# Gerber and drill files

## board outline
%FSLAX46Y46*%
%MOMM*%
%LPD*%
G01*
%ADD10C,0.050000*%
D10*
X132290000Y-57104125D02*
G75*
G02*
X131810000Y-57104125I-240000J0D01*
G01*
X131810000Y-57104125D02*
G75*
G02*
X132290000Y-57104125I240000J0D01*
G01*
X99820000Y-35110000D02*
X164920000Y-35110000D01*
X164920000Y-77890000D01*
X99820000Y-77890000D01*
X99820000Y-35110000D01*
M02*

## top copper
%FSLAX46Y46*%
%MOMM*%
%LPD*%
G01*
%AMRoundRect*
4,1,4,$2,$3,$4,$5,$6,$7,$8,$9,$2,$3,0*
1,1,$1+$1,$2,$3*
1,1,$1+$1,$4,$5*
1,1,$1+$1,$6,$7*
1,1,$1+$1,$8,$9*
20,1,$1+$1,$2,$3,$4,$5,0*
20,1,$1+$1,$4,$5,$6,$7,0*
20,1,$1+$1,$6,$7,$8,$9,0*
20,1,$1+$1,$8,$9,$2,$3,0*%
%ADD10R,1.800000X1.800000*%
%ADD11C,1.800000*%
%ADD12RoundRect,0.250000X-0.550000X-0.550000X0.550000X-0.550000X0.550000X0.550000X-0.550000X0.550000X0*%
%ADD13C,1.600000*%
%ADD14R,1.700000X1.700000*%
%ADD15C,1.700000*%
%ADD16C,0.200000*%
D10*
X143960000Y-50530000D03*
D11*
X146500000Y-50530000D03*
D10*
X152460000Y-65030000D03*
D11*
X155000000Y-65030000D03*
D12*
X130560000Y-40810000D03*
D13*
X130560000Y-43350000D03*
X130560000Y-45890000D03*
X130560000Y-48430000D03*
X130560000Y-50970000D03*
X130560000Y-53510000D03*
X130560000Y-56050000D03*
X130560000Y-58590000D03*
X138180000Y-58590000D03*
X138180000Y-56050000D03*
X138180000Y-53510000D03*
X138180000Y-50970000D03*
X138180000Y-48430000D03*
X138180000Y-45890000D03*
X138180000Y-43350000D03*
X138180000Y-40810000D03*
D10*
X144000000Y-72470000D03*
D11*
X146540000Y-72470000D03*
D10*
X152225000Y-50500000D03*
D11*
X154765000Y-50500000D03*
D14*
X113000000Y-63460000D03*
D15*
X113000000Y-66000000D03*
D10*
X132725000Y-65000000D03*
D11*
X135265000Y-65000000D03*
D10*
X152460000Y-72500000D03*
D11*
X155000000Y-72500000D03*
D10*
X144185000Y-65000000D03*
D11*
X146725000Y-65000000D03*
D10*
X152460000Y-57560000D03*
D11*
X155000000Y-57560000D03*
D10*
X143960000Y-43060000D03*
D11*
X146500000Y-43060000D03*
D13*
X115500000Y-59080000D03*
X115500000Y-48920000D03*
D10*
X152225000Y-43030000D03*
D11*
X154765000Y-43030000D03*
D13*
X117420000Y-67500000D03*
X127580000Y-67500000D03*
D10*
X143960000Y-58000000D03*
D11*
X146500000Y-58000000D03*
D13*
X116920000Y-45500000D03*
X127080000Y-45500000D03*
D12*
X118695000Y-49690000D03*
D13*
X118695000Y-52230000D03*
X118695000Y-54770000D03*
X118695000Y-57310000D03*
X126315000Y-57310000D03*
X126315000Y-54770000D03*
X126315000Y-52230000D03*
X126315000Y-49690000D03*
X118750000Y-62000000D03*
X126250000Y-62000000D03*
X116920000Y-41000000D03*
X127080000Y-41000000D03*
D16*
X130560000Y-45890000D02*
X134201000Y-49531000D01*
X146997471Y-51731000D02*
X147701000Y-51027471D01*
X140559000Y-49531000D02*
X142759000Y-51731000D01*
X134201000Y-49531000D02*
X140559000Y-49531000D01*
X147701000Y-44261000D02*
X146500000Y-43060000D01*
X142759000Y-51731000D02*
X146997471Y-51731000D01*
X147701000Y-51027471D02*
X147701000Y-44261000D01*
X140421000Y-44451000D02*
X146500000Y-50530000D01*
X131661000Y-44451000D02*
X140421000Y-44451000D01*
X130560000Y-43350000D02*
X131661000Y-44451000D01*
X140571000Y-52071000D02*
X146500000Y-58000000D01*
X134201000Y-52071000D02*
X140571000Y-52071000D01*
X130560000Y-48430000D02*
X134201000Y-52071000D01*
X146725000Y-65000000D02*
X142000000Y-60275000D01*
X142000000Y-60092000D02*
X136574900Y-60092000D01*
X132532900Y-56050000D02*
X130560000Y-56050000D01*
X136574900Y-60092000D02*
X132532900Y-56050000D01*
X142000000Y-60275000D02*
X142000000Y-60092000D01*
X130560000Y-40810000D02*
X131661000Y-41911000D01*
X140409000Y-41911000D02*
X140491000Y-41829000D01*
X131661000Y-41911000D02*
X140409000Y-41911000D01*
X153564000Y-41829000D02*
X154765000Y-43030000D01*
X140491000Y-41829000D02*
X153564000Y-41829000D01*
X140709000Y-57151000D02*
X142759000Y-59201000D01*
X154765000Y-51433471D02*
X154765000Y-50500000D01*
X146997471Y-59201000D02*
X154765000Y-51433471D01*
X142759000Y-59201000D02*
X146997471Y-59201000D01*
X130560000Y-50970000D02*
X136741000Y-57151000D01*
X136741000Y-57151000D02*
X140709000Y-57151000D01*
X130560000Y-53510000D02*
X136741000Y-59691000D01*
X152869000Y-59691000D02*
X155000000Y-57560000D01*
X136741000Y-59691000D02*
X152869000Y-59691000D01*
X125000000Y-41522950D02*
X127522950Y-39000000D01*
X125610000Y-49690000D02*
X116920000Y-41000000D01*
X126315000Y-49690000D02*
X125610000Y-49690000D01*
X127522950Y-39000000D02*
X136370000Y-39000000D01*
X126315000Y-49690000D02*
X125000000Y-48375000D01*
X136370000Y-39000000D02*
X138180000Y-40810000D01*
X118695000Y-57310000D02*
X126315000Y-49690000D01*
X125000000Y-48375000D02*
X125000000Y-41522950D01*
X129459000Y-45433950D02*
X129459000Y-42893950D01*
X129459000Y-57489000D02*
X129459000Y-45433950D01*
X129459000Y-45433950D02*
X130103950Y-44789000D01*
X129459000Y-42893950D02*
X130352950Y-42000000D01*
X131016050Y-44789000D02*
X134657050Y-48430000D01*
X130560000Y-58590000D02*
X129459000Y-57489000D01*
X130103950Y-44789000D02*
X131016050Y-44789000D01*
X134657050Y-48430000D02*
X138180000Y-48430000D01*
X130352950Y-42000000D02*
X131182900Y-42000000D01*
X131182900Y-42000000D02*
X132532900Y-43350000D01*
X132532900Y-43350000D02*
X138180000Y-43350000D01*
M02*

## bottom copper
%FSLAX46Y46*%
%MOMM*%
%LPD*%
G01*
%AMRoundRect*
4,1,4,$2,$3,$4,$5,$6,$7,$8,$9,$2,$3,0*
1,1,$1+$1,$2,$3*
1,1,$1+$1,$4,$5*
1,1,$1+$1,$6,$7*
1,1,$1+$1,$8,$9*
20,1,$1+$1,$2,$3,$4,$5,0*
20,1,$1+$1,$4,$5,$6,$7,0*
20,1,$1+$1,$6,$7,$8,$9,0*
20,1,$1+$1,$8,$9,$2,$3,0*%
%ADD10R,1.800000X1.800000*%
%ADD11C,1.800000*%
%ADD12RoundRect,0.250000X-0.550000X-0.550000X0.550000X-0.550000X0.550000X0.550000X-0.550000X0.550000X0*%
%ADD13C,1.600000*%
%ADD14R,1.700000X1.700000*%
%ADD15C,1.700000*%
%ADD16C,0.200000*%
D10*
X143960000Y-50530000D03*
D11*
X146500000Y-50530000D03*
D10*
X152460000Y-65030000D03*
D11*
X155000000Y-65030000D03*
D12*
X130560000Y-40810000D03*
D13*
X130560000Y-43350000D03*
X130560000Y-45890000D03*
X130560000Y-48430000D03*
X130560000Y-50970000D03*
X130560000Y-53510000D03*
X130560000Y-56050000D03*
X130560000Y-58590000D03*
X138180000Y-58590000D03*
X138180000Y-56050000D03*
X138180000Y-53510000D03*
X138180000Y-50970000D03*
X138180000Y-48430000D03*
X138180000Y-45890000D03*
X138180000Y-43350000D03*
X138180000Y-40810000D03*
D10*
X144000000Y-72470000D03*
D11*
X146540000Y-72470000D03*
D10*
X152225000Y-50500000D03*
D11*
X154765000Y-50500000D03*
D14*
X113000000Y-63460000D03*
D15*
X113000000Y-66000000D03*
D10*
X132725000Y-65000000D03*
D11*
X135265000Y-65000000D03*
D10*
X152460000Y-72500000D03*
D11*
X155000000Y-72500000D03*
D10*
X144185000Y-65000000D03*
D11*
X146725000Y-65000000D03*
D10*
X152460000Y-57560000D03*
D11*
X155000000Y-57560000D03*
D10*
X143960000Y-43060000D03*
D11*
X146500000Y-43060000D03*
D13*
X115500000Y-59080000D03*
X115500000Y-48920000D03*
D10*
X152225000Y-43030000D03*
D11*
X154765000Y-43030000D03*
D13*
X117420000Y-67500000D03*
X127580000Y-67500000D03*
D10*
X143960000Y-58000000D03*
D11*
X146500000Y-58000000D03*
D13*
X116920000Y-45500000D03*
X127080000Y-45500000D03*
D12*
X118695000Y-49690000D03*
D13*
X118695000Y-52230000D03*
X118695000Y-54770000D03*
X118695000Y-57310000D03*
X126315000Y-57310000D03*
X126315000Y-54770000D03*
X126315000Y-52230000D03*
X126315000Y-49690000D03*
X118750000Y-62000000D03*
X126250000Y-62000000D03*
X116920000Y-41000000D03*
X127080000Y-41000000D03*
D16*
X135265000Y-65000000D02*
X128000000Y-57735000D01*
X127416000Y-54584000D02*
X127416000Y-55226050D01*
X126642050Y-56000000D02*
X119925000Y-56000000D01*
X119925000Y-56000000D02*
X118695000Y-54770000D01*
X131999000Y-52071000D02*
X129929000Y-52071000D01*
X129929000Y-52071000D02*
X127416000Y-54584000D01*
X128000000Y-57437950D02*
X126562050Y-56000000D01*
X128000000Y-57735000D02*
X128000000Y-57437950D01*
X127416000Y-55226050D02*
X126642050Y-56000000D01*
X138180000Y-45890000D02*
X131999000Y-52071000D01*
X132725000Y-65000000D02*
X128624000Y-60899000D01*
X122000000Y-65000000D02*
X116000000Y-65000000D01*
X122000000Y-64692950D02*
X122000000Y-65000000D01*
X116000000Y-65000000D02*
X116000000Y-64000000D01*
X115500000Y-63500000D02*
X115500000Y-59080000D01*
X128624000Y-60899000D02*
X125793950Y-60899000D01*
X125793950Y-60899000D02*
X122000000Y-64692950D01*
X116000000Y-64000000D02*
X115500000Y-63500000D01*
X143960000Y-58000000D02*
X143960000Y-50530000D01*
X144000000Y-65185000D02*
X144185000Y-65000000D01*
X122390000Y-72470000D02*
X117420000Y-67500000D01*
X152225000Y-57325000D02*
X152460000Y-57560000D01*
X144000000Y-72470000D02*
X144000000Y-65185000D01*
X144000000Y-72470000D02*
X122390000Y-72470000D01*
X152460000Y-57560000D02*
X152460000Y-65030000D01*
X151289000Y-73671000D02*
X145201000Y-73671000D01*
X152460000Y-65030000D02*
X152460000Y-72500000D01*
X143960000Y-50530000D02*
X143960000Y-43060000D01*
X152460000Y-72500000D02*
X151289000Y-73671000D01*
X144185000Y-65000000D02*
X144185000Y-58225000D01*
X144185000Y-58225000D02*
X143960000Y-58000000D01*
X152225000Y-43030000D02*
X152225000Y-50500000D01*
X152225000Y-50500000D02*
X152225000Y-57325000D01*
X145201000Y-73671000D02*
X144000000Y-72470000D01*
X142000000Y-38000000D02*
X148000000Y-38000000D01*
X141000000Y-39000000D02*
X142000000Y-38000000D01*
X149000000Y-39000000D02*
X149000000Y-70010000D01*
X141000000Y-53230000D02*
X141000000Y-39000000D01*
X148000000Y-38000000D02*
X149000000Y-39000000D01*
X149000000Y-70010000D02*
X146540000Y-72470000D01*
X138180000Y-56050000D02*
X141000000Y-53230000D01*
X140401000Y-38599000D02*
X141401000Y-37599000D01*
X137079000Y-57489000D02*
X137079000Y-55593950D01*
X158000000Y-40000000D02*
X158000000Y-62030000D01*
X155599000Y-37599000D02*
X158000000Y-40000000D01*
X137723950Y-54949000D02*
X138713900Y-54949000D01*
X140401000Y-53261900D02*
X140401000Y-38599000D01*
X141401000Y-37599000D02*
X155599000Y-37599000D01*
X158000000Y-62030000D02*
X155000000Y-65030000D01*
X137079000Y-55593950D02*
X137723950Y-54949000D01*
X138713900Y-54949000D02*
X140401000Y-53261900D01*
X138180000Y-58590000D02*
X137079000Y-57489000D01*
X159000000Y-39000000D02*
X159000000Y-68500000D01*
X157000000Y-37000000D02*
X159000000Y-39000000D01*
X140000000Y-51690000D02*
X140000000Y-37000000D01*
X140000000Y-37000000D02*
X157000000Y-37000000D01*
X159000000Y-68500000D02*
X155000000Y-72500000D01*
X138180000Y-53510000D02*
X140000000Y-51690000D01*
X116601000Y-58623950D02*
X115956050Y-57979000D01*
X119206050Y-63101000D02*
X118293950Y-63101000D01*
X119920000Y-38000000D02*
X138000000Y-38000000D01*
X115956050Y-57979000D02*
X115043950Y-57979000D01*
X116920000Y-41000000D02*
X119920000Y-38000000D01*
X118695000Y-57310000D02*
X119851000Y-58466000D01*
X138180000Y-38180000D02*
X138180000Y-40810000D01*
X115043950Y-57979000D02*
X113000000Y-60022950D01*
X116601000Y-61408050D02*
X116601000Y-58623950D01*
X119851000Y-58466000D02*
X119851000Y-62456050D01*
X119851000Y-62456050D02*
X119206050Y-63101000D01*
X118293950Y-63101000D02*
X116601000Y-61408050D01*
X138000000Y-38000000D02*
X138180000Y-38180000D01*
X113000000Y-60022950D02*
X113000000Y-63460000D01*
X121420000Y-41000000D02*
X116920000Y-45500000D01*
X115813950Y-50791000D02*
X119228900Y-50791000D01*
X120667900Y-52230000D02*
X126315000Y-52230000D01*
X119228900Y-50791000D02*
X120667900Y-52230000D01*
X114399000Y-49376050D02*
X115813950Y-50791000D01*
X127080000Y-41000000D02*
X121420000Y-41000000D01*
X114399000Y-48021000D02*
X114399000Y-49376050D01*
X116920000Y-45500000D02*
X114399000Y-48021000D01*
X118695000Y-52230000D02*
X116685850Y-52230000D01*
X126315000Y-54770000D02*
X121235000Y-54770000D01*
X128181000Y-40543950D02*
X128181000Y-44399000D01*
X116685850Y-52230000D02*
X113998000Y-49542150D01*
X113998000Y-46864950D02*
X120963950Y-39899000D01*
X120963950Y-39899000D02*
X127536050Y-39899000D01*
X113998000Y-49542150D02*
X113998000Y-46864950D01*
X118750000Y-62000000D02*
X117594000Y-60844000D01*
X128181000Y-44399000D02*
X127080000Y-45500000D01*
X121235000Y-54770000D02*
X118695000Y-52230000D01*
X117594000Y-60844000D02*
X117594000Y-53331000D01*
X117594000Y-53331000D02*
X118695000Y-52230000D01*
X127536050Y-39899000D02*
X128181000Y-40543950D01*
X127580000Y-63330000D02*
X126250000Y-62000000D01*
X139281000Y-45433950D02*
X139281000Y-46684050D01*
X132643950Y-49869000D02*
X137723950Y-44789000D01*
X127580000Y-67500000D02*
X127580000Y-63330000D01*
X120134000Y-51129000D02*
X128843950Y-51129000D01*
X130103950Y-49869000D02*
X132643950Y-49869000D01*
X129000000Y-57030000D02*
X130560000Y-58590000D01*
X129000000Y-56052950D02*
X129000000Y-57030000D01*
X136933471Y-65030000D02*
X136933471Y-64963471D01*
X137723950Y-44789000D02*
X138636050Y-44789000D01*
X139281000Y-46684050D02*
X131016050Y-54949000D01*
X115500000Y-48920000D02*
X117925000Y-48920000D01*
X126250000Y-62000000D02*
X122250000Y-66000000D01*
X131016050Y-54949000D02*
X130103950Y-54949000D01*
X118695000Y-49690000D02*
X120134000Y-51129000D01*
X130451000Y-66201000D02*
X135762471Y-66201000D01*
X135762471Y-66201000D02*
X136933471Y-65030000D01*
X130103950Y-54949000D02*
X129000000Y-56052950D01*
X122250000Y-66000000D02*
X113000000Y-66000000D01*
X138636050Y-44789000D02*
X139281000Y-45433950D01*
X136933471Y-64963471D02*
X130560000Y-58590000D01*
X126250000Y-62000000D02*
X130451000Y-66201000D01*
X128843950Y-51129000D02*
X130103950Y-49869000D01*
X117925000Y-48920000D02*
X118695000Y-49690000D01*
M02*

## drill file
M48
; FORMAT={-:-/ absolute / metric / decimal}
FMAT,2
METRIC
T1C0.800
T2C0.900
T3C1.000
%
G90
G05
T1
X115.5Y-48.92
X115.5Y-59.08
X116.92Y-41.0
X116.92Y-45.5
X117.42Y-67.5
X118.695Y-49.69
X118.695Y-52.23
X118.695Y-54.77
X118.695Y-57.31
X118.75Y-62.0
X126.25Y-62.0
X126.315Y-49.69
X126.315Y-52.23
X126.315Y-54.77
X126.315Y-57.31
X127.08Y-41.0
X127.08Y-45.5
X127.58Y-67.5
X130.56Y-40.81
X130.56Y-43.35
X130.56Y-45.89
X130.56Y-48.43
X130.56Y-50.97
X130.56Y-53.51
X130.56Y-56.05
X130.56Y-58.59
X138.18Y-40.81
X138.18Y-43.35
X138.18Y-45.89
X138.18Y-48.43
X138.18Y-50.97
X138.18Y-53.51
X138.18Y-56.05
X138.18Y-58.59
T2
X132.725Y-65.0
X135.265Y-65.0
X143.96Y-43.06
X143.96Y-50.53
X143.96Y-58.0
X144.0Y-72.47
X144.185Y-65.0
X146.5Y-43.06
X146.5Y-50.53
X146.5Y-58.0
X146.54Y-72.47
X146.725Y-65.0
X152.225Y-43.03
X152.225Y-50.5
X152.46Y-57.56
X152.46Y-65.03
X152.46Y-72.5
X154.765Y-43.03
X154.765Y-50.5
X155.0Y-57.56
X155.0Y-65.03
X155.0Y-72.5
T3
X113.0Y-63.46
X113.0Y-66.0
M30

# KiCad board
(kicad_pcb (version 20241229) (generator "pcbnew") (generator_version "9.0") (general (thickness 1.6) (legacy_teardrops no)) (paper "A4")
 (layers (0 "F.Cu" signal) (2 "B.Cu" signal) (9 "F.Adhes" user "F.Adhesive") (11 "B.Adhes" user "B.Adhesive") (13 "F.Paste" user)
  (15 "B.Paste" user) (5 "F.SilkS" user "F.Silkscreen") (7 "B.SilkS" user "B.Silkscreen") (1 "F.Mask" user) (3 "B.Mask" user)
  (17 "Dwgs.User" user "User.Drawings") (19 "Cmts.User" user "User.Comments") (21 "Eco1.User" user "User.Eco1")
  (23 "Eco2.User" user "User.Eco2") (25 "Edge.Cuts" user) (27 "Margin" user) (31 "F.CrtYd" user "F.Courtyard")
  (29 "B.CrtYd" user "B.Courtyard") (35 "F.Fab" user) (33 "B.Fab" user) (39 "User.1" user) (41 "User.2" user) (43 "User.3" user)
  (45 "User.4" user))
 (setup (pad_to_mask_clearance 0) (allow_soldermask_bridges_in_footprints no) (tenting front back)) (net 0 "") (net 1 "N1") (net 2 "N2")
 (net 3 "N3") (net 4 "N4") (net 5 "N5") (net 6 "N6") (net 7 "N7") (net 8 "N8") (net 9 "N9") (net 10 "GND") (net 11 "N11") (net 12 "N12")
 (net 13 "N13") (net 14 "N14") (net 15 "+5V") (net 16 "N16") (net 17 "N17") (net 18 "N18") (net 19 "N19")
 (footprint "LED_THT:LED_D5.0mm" (layer "F.Cu") (at 143.96 50.53)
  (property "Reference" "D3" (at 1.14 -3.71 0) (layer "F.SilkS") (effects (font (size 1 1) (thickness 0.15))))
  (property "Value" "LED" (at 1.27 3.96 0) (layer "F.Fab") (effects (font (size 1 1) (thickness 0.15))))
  (pad "1" thru_hole rect (at 0 0) (size 1.8 1.8) (drill 0.9) (layers "*.Cu" "*.Mask") (remove_unused_layers no) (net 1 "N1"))
  (pad "2" thru_hole circle (at 2.54 0) (size 1.8 1.8) (drill 0.9) (layers "*.Cu" "*.Mask") (remove_unused_layers no) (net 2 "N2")))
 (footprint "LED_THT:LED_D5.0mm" (layer "F.Cu") (at 152.46 65.03)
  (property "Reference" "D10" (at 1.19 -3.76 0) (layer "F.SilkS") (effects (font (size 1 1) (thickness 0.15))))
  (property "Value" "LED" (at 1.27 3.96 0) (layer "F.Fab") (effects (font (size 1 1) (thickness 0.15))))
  (pad "1" thru_hole rect (at 0 0) (size 1.8 1.8) (drill 0.9) (layers "*.Cu" "*.Mask") (remove_unused_layers no) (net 1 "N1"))
  (pad "2" thru_hole circle (at 2.54 0) (size 1.8 1.8) (drill 0.9) (layers "*.Cu" "*.Mask") (remove_unused_layers no) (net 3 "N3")))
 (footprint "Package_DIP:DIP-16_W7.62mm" (layer "F.Cu") (at 130.56 40.81)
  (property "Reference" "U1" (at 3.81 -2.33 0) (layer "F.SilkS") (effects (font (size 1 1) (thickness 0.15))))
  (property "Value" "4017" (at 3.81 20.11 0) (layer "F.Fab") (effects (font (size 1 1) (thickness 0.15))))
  (pad "1" thru_hole roundrect (at 0 0) (size 1.6 1.6) (drill 0.8) (layers "*.Cu" "*.Mask") (remove_unused_layers no)
   (roundrect_rratio 0.15625) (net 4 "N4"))
  (pad "2" thru_hole circle (at 0 2.54) (size 1.6 1.6) (drill 0.8) (layers "*.Cu" "*.Mask") (remove_unused_layers no) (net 2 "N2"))
  (pad "3" thru_hole circle (at 0 5.08) (size 1.6 1.6) (drill 0.8) (layers "*.Cu" "*.Mask") (remove_unused_layers no) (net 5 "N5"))
  (pad "4" thru_hole circle (at 0 7.62) (size 1.6 1.6) (drill 0.8) (layers "*.Cu" "*.Mask") (remove_unused_layers no) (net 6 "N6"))
  (pad "5" thru_hole circle (at 0 10.16) (size 1.6 1.6) (drill 0.8) (layers "*.Cu" "*.Mask") (remove_unused_layers no) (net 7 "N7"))
  (pad "6" thru_hole circle (at 0 12.7) (size 1.6 1.6) (drill 0.8) (layers "*.Cu" "*.Mask") (remove_unused_layers no) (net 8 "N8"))
  (pad "7" thru_hole circle (at 0 15.24) (size 1.6 1.6) (drill 0.8) (layers "*.Cu" "*.Mask") (remove_unused_layers no) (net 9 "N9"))
  (pad "8" thru_hole circle (at 0 17.78) (size 1.6 1.6) (drill 0.8) (layers "*.Cu" "*.Mask") (remove_unused_layers no) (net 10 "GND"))
  (pad "9" thru_hole circle (at 7.62 17.78) (size 1.6 1.6) (drill 0.8) (layers "*.Cu" "*.Mask") (remove_unused_layers no) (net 3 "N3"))
  (pad "10" thru_hole circle (at 7.62 15.24) (size 1.6 1.6) (drill 0.8) (layers "*.Cu" "*.Mask") (remove_unused_layers no) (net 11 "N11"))
  (pad "11" thru_hole circle (at 7.62 12.7) (size 1.6 1.6) (drill 0.8) (layers "*.Cu" "*.Mask") (remove_unused_layers no) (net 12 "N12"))
  (pad "12" thru_hole circle (at 7.62 10.16) (size 1.6 1.6) (drill 0.8) (layers "*.Cu" "*.Mask") (remove_unused_layers no) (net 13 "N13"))
  (pad "13" thru_hole circle (at 7.62 7.62) (size 1.6 1.6) (drill 0.8) (layers "*.Cu" "*.Mask") (remove_unused_layers no) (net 10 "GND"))
  (pad "14" thru_hole circle (at 7.62 5.08) (size 1.6 1.6) (drill 0.8) (layers "*.Cu" "*.Mask") (remove_unused_layers no) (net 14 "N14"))
  (pad "15" thru_hole circle (at 7.62 2.54) (size 1.6 1.6) (drill 0.8) (layers "*.Cu" "*.Mask") (remove_unused_layers no) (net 10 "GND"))
  (pad "16" thru_hole circle (at 7.62 0) (size 1.6 1.6) (drill 0.8) (layers "*.Cu" "*.Mask") (remove_unused_layers no) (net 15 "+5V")))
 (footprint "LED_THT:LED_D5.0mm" (layer "F.Cu") (at 144 72.47)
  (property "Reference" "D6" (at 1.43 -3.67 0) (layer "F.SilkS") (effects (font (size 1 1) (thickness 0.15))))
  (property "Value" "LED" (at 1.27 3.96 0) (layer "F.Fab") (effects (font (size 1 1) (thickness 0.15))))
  (pad "1" thru_hole rect (at 0 0) (size 1.8 1.8) (drill 0.9) (layers "*.Cu" "*.Mask") (remove_unused_layers no) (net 1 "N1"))
  (pad "2" thru_hole circle (at 2.54 0) (size 1.8 1.8) (drill 0.9) (layers "*.Cu" "*.Mask") (remove_unused_layers no) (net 11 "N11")))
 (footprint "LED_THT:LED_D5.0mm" (layer "F.Cu") (at 152.225 50.5)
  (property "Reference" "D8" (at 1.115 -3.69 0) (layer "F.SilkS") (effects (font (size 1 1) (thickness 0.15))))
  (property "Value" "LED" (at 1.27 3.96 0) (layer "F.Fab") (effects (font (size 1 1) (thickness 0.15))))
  (pad "1" thru_hole rect (at 0 0) (size 1.8 1.8) (drill 0.9) (layers "*.Cu" "*.Mask") (remove_unused_layers no) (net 1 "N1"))
  (pad "2" thru_hole circle (at 2.54 0) (size 1.8 1.8) (drill 0.9) (layers "*.Cu" "*.Mask") (remove_unused_layers no) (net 7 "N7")))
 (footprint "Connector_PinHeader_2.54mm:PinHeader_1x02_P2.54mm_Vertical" (layer "F.Cu") (at 113 63.46)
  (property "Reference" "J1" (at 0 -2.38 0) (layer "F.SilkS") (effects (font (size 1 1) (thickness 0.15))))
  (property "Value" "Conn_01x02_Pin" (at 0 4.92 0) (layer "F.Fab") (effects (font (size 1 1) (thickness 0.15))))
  (pad "1" thru_hole rect (at 0 0) (size 1.7 1.7) (drill 1) (layers "*.Cu" "*.Mask") (remove_unused_layers no) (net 15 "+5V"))
  (pad "2" thru_hole circle (at 0 2.54) (size 1.7 1.7) (drill 1) (layers "*.Cu" "*.Mask") (remove_unused_layers no) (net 10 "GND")))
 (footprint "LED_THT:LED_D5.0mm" (layer "F.Cu") (at 132.725 65)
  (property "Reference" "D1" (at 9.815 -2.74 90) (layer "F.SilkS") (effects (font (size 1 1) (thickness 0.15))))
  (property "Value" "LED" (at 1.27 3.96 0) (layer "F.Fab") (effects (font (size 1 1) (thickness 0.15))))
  (pad "1" thru_hole rect (at 0 0) (size 1.8 1.8) (drill 0.9) (layers "*.Cu" "*.Mask") (remove_unused_layers no) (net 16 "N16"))
  (pad "2" thru_hole circle (at 2.54 0) (size 1.8 1.8) (drill 0.9) (layers "*.Cu" "*.Mask") (remove_unused_layers no) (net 14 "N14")))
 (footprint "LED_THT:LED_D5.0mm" (layer "F.Cu") (at 152.46 72.5)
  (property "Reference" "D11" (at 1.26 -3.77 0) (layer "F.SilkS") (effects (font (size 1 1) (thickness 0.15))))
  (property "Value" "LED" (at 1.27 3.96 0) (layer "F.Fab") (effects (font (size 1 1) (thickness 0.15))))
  (pad "1" thru_hole rect (at 0 0) (size 1.8 1.8) (drill 0.9) (layers "*.Cu" "*.Mask") (remove_unused_layers no) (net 1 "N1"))
  (pad "2" thru_hole circle (at 2.54 0) (size 1.8 1.8) (drill 0.9) (layers "*.Cu" "*.Mask") (remove_unused_layers no) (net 12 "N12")))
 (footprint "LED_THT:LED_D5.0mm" (layer "F.Cu") (at 144.185 65)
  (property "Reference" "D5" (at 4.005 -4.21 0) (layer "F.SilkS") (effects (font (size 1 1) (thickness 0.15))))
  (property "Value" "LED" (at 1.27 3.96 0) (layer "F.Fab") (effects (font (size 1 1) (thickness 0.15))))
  (pad "1" thru_hole rect (at 0 0) (size 1.8 1.8) (drill 0.9) (layers "*.Cu" "*.Mask") (remove_unused_layers no) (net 1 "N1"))
  (pad "2" thru_hole circle (at 2.54 0) (size 1.8 1.8) (drill 0.9) (layers "*.Cu" "*.Mask") (remove_unused_layers no) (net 9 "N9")))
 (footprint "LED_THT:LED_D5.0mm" (layer "F.Cu") (at 152.46 57.56)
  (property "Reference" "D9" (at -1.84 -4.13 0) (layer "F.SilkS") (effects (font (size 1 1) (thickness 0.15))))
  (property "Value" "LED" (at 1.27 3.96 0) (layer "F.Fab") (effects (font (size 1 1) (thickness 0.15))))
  (pad "1" thru_hole rect (at 0 0) (size 1.8 1.8) (drill 0.9) (layers "*.Cu" "*.Mask") (remove_unused_layers no) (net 1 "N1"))
  (pad "2" thru_hole circle (at 2.54 0) (size 1.8 1.8) (drill 0.9) (layers "*.Cu" "*.Mask") (remove_unused_layers no) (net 8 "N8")))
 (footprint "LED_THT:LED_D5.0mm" (layer "F.Cu") (at 143.96 43.06)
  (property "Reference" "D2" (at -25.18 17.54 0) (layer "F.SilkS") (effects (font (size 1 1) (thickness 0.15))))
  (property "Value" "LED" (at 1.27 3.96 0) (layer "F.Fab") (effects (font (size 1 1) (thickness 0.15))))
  (pad "1" thru_hole rect (at 0 0) (size 1.8 1.8) (drill 0.9) (layers "*.Cu" "*.Mask") (remove_unused_layers no) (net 1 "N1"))
  (pad "2" thru_hole circle (at 2.54 0) (size 1.8 1.8) (drill 0.9) (layers "*.Cu" "*.Mask") (remove_unused_layers no) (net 5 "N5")))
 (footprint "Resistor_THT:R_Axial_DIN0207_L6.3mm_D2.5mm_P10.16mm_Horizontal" (layer "F.Cu") (at 115.5 59.08 90)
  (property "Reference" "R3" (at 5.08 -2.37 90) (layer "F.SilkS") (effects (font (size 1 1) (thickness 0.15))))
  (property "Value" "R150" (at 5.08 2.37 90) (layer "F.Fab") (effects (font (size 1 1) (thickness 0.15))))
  (pad "1" thru_hole circle (at 0 0 90) (size 1.6 1.6) (drill 0.8) (layers "*.Cu" "*.Mask") (remove_unused_layers no) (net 16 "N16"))
  (pad "2" thru_hole circle (at 10.16 0 90) (size 1.6 1.6) (drill 0.8) (layers "*.Cu" "*.Mask") (remove_unused_layers no) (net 10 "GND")))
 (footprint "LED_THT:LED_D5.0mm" (layer "F.Cu") (at 152.225 43.03)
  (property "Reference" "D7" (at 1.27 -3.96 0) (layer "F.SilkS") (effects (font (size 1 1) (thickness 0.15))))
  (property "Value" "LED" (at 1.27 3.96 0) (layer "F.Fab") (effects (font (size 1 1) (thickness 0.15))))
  (pad "1" thru_hole rect (at 0 0) (size 1.8 1.8) (drill 0.9) (layers "*.Cu" "*.Mask") (remove_unused_layers no) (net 1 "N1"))
  (pad "2" thru_hole circle (at 2.54 0) (size 1.8 1.8) (drill 0.9) (layers "*.Cu" "*.Mask") (remove_unused_layers no) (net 4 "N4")))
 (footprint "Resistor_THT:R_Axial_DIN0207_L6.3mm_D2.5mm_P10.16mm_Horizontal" (layer "F.Cu") (at 117.42 67.5)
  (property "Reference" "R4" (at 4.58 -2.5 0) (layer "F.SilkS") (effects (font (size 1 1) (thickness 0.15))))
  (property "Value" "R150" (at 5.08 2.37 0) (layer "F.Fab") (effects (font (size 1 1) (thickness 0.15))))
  (pad "1" thru_hole circle (at 0 0) (size 1.6 1.6) (drill 0.8) (layers "*.Cu" "*.Mask") (remove_unused_layers no) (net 1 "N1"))
  (pad "2" thru_hole circle (at 10.16 0) (size 1.6 1.6) (drill 0.8) (layers "*.Cu" "*.Mask") (remove_unused_layers no) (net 10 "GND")))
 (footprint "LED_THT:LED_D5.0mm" (layer "F.Cu") (at 143.96 58)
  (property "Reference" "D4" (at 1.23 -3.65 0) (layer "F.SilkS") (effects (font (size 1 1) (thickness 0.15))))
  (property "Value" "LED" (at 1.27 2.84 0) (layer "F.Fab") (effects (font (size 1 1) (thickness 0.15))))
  (pad "1" thru_hole rect (at 0 0) (size 1.8 1.8) (drill 0.9) (layers "*.Cu" "*.Mask") (remove_unused_layers no) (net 1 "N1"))
  (pad "2" thru_hole circle (at 2.54 0) (size 1.8 1.8) (drill 0.9) (layers "*.Cu" "*.Mask") (remove_unused_layers no) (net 6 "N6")))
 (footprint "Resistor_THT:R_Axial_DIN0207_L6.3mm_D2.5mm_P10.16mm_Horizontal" (layer "F.Cu") (at 116.92 45.5)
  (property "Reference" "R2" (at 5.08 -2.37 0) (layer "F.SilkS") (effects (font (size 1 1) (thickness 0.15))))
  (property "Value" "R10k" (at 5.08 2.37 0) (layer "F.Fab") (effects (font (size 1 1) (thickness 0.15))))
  (pad "1" thru_hole circle (at 0 0) (size 1.6 1.6) (drill 0.8) (layers "*.Cu" "*.Mask") (remove_unused_layers no) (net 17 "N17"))
  (pad "2" thru_hole circle (at 10.16 0) (size 1.6 1.6) (drill 0.8) (layers "*.Cu" "*.Mask") (remove_unused_layers no) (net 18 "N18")))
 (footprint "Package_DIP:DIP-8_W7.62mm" (layer "F.Cu") (at 118.695 49.69)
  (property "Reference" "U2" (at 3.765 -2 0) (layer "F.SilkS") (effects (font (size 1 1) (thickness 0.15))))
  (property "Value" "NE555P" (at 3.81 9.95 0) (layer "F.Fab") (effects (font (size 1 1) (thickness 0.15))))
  (pad "1" thru_hole roundrect (at 0 0) (size 1.6 1.6) (drill 0.8) (layers "*.Cu" "*.Mask") (remove_unused_layers no)
   (roundrect_rratio 0.15625) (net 10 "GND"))
  (pad "2" thru_hole circle (at 0 2.54) (size 1.6 1.6) (drill 0.8) (layers "*.Cu" "*.Mask") (remove_unused_layers no) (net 18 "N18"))
  (pad "3" thru_hole circle (at 0 5.08) (size 1.6 1.6) (drill 0.8) (layers "*.Cu" "*.Mask") (remove_unused_layers no) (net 14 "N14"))
  (pad "4" thru_hole circle (at 0 7.62) (size 1.6 1.6) (drill 0.8) (layers "*.Cu" "*.Mask") (remove_unused_layers no) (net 15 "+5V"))
  (pad "5" thru_hole circle (at 7.62 7.62) (size 1.6 1.6) (drill 0.8) (layers "*.Cu" "*.Mask") (remove_unused_layers no) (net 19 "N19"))
  (pad "6" thru_hole circle (at 7.62 5.08) (size 1.6 1.6) (drill 0.8) (layers "*.Cu" "*.Mask") (remove_unused_layers no) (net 18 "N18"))
  (pad "7" thru_hole circle (at 7.62 2.54) (size 1.6 1.6) (drill 0.8) (layers "*.Cu" "*.Mask") (remove_unused_layers no) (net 17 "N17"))
  (pad "8" thru_hole circle (at 7.62 0) (size 1.6 1.6) (drill 0.8) (layers "*.Cu" "*.Mask") (remove_unused_layers no) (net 15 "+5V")))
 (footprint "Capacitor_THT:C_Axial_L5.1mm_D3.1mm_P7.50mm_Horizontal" (layer "F.Cu") (at 118.75 62)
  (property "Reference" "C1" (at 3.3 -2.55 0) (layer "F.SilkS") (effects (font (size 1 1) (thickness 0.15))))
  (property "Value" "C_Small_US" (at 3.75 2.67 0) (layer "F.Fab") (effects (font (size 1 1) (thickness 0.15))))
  (pad "1" thru_hole circle (at 0 0) (size 1.6 1.6) (drill 0.8) (layers "*.Cu" "*.Mask") (remove_unused_layers no) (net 18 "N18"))
  (pad "2" thru_hole circle (at 7.5 0) (size 1.6 1.6) (drill 0.8) (layers "*.Cu" "*.Mask") (remove_unused_layers no) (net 10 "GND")))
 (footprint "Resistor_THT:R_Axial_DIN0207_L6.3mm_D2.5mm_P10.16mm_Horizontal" (layer "F.Cu") (at 116.92 41)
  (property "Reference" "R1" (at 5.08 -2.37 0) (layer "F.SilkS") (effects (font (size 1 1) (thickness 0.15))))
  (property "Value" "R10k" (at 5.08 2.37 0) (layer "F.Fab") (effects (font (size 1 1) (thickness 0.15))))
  (pad "1" thru_hole circle (at 0 0) (size 1.6 1.6) (drill 0.8) (layers "*.Cu" "*.Mask") (remove_unused_layers no) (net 15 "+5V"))
  (pad "2" thru_hole circle (at 10.16 0) (size 1.6 1.6) (drill 0.8) (layers "*.Cu" "*.Mask") (remove_unused_layers no) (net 17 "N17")))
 (gr_circle (center 132.05 57.104125) (end 132.29 57.104125) (stroke (width 0.05) (type default)) (fill no) (layer "Edge.Cuts"))
 (gr_rect (start 99.82 35.11) (end 164.92 77.89) (stroke (width 0.05) (type default)) (fill no) (layer "Edge.Cuts"))
 (segment (start 135.265 65) (end 128 57.735) (width 0.2) (layer "B.Cu") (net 14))
 (segment (start 127.416 54.584) (end 127.416 55.22605) (width 0.2) (layer "B.Cu") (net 14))
 (segment (start 126.64205 56) (end 119.925 56) (width 0.2) (layer "B.Cu") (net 14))
 (segment (start 119.925 56) (end 118.695 54.77) (width 0.2) (layer "B.Cu") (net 14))
 (segment (start 131.999 52.071) (end 129.929 52.071) (width 0.2) (layer "B.Cu") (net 14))
 (segment (start 129.929 52.071) (end 127.416 54.584) (width 0.2) (layer "B.Cu") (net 14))
 (segment (start 128 57.43795) (end 126.56205 56) (width 0.2) (layer "B.Cu") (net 14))
 (segment (start 128 57.735) (end 128 57.43795) (width 0.2) (layer "B.Cu") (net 14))
 (segment (start 127.416 55.22605) (end 126.64205 56) (width 0.2) (layer "B.Cu") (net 14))
 (segment (start 138.18 45.89) (end 131.999 52.071) (width 0.2) (layer "B.Cu") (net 14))
 (segment (start 132.725 65) (end 128.624 60.899) (width 0.2) (layer "B.Cu") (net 16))
 (segment (start 122 65) (end 116 65) (width 0.2) (layer "B.Cu") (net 16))
 (segment (start 122 64.69295) (end 122 65) (width 0.2) (layer "B.Cu") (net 16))
 (segment (start 116 65) (end 116 64) (width 0.2) (layer "B.Cu") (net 16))
 (segment (start 115.5 63.5) (end 115.5 59.08) (width 0.2) (layer "B.Cu") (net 16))
 (segment (start 128.624 60.899) (end 125.79395 60.899) (width 0.2) (layer "B.Cu") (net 16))
 (segment (start 125.79395 60.899) (end 122 64.69295) (width 0.2) (layer "B.Cu") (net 16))
 (segment (start 116 64) (end 115.5 63.5) (width 0.2) (layer "B.Cu") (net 16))
 (segment (start 143.96 58) (end 143.96 50.53) (width 0.2) (layer "B.Cu") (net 1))
 (segment (start 144 65.185) (end 144.185 65) (width 0.2) (layer "B.Cu") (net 1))
 (segment (start 122.39 72.47) (end 117.42 67.5) (width 0.2) (layer "B.Cu") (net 1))
 (segment (start 152.225 57.325) (end 152.46 57.56) (width 0.2) (layer "B.Cu") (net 1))
 (segment (start 144 72.47) (end 144 65.185) (width 0.2) (layer "B.Cu") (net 1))
 (segment (start 144 72.47) (end 122.39 72.47) (width 0.2) (layer "B.Cu") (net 1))
 (segment (start 152.46 57.56) (end 152.46 65.03) (width 0.2) (layer "B.Cu") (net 1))
 (segment (start 151.289 73.671) (end 145.201 73.671) (width 0.2) (layer "B.Cu") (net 1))
 (segment (start 152.46 65.03) (end 152.46 72.5) (width 0.2) (layer "B.Cu") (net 1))
 (segment (start 143.96 50.53) (end 143.96 43.06) (width 0.2) (layer "B.Cu") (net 1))
 (segment (start 152.46 72.5) (end 151.289 73.671) (width 0.2) (layer "B.Cu") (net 1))
 (segment (start 144.185 65) (end 144.185 58.225) (width 0.2) (layer "B.Cu") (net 1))
 (segment (start 144.185 58.225) (end 143.96 58) (width 0.2) (layer "B.Cu") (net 1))
 (segment (start 152.225 43.03) (end 152.225 50.5) (width 0.2) (layer "B.Cu") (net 1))
 (segment (start 152.225 50.5) (end 152.225 57.325) (width 0.2) (layer "B.Cu") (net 1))
 (segment (start 145.201 73.671) (end 144 72.47) (width 0.2) (layer "B.Cu") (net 1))
 (segment (start 130.56 45.89) (end 134.201 49.531) (width 0.2) (layer "F.Cu") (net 5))
 (segment (start 146.997471 51.731) (end 147.701 51.027471) (width 0.2) (layer "F.Cu") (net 5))
 (segment (start 140.559 49.531) (end 142.759 51.731) (width 0.2) (layer "F.Cu") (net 5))
 (segment (start 134.201 49.531) (end 140.559 49.531) (width 0.2) (layer "F.Cu") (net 5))
 (segment (start 147.701 44.261) (end 146.5 43.06) (width 0.2) (layer "F.Cu") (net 5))
 (segment (start 142.759 51.731) (end 146.997471 51.731) (width 0.2) (layer "F.Cu") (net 5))
 (segment (start 147.701 51.027471) (end 147.701 44.261) (width 0.2) (layer "F.Cu") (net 5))
 (segment (start 140.421 44.451) (end 146.5 50.53) (width 0.2) (layer "F.Cu") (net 2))
 (segment (start 131.661 44.451) (end 140.421 44.451) (width 0.2) (layer "F.Cu") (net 2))
 (segment (start 130.56 43.35) (end 131.661 44.451) (width 0.2) (layer "F.Cu") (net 2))
 (segment (start 140.571 52.071) (end 146.5 58) (width 0.2) (layer "F.Cu") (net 6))
 (segment (start 134.201 52.071) (end 140.571 52.071) (width 0.2) (layer "F.Cu") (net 6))
 (segment (start 130.56 48.43) (end 134.201 52.071) (width 0.2) (layer "F.Cu") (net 6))
 (segment (start 146.725 65) (end 142 60.275) (width 0.2) (layer "F.Cu") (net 9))
 (segment (start 142 60.092) (end 136.5749 60.092) (width 0.2) (layer "F.Cu") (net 9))
 (segment (start 132.5329 56.05) (end 130.56 56.05) (width 0.2) (layer "F.Cu") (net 9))
 (segment (start 136.5749 60.092) (end 132.5329 56.05) (width 0.2) (layer "F.Cu") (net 9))
 (segment (start 142 60.275) (end 142 60.092) (width 0.2) (layer "F.Cu") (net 9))
 (segment (start 142 38) (end 148 38) (width 0.2) (layer "B.Cu") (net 11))
 (segment (start 141 39) (end 142 38) (width 0.2) (layer "B.Cu") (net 11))
 (segment (start 149 39) (end 149 70.01) (width 0.2) (layer "B.Cu") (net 11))
 (segment (start 141 53.23) (end 141 39) (width 0.2) (layer "B.Cu") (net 11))
 (segment (start 148 38) (end 149 39) (width 0.2) (layer "B.Cu") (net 11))
 (segment (start 149 70.01) (end 146.54 72.47) (width 0.2) (layer "B.Cu") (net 11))
 (segment (start 138.18 56.05) (end 141 53.23) (width 0.2) (layer "B.Cu") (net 11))
 (segment (start 130.56 40.81) (end 131.661 41.911) (width 0.2) (layer "F.Cu") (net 4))
 (segment (start 140.409 41.911) (end 140.491 41.829) (width 0.2) (layer "F.Cu") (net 4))
 (segment (start 131.661 41.911) (end 140.409 41.911) (width 0.2) (layer "F.Cu") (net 4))
 (segment (start 153.564 41.829) (end 154.765 43.03) (width 0.2) (layer "F.Cu") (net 4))
 (segment (start 140.491 41.829) (end 153.564 41.829) (width 0.2) (layer "F.Cu") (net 4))
 (segment (start 140.709 57.151) (end 142.759 59.201) (width 0.2) (layer "F.Cu") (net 7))
 (segment (start 154.765 51.433471) (end 154.765 50.5) (width 0.2) (layer "F.Cu") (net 7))
 (segment (start 146.997471 59.201) (end 154.765 51.433471) (width 0.2) (layer "F.Cu") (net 7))
 (segment (start 142.759 59.201) (end 146.997471 59.201) (width 0.2) (layer "F.Cu") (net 7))
 (segment (start 130.56 50.97) (end 136.741 57.151) (width 0.2) (layer "F.Cu") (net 7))
 (segment (start 136.741 57.151) (end 140.709 57.151) (width 0.2) (layer "F.Cu") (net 7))
 (segment (start 130.56 53.51) (end 136.741 59.691) (width 0.2) (layer "F.Cu") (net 8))
 (segment (start 152.869 59.691) (end 155 57.56) (width 0.2) (layer "F.Cu") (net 8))
 (segment (start 136.741 59.691) (end 152.869 59.691) (width 0.2) (layer "F.Cu") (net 8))
 (segment (start 140.401 38.599) (end 141.401 37.599) (width 0.2) (layer "B.Cu") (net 3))
 (segment (start 137.079 57.489) (end 137.079 55.59395) (width 0.2) (layer "B.Cu") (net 3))
 (segment (start 158 40) (end 158 62.03) (width 0.2) (layer "B.Cu") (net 3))
 (segment (start 155.599 37.599) (end 158 40) (width 0.2) (layer "B.Cu") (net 3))
 (segment (start 137.72395 54.949) (end 138.7139 54.949) (width 0.2) (layer "B.Cu") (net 3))
 (segment (start 140.401 53.2619) (end 140.401 38.599) (width 0.2) (layer "B.Cu") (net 3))
 (segment (start 141.401 37.599) (end 155.599 37.599) (width 0.2) (layer "B.Cu") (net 3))
 (segment (start 158 62.03) (end 155 65.03) (width 0.2) (layer "B.Cu") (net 3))
 (segment (start 137.079 55.59395) (end 137.72395 54.949) (width 0.2) (layer "B.Cu") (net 3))
 (segment (start 138.7139 54.949) (end 140.401 53.2619) (width 0.2) (layer "B.Cu") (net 3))
 (segment (start 138.18 58.59) (end 137.079 57.489) (width 0.2) (layer "B.Cu") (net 3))
 (segment (start 159 39) (end 159 68.5) (width 0.2) (layer "B.Cu") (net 12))
 (segment (start 157 37) (end 159 39) (width 0.2) (layer "B.Cu") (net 12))
 (segment (start 140 51.69) (end 140 37) (width 0.2) (layer "B.Cu") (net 12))
 (segment (start 140 37) (end 157 37) (width 0.2) (layer "B.Cu") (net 12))
 (segment (start 159 68.5) (end 155 72.5) (width 0.2) (layer "B.Cu") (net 12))
 (segment (start 138.18 53.51) (end 140 51.69) (width 0.2) (layer "B.Cu") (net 12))
 (segment (start 125 41.52295) (end 127.52295 39) (width 0.2) (layer "F.Cu") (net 15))
 (segment (start 125.61 49.69) (end 116.92 41) (width 0.2) (layer "F.Cu") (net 15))
 (segment (start 126.315 49.69) (end 125.61 49.69) (width 0.2) (layer "F.Cu") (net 15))
 (segment (start 127.52295 39) (end 136.37 39) (width 0.2) (layer "F.Cu") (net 15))
 (segment (start 126.315 49.69) (end 125 48.375) (width 0.2) (layer "F.Cu") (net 15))
 (segment (start 136.37 39) (end 138.18 40.81) (width 0.2) (layer "F.Cu") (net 15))
 (segment (start 118.695 57.31) (end 126.315 49.69) (width 0.2) (layer "F.Cu") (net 15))
 (segment (start 125 48.375) (end 125 41.52295) (width 0.2) (layer "F.Cu") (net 15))
 (segment (start 116.601 58.62395) (end 115.95605 57.979) (width 0.2) (layer "B.Cu") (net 15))
 (segment (start 119.20605 63.101) (end 118.29395 63.101) (width 0.2) (layer "B.Cu") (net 15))
 (segment (start 119.92 38) (end 138 38) (width 0.2) (layer "B.Cu") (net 15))
 (segment (start 115.95605 57.979) (end 115.04395 57.979) (width 0.2) (layer "B.Cu") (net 15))
 (segment (start 116.92 41) (end 119.92 38) (width 0.2) (layer "B.Cu") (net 15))
 (segment (start 118.695 57.31) (end 119.851 58.466) (width 0.2) (layer "B.Cu") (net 15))
 (segment (start 138.18 38.18) (end 138.18 40.81) (width 0.2) (layer "B.Cu") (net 15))
 (segment (start 115.04395 57.979) (end 113 60.02295) (width 0.2) (layer "B.Cu") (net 15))
 (segment (start 116.601 61.40805) (end 116.601 58.62395) (width 0.2) (layer "B.Cu") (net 15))
 (segment (start 119.851 58.466) (end 119.851 62.45605) (width 0.2) (layer "B.Cu") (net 15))
 (segment (start 119.851 62.45605) (end 119.20605 63.101) (width 0.2) (layer "B.Cu") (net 15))
 (segment (start 118.29395 63.101) (end 116.601 61.40805) (width 0.2) (layer "B.Cu") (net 15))
 (segment (start 138 38) (end 138.18 38.18) (width 0.2) (layer "B.Cu") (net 15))
 (segment (start 113 60.02295) (end 113 63.46) (width 0.2) (layer "B.Cu") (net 15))
 (segment (start 121.42 41) (end 116.92 45.5) (width 0.2) (layer "B.Cu") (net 17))
 (segment (start 115.81395 50.791) (end 119.2289 50.791) (width 0.2) (layer "B.Cu") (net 17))
 (segment (start 120.6679 52.23) (end 126.315 52.23) (width 0.2) (layer "B.Cu") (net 17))
 (segment (start 119.2289 50.791) (end 120.6679 52.23) (width 0.2) (layer "B.Cu") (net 17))
 (segment (start 114.399 49.37605) (end 115.81395 50.791) (width 0.2) (layer "B.Cu") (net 17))
 (segment (start 127.08 41) (end 121.42 41) (width 0.2) (layer "B.Cu") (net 17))
 (segment (start 114.399 48.021) (end 114.399 49.37605) (width 0.2) (layer "B.Cu") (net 17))
 (segment (start 116.92 45.5) (end 114.399 48.021) (width 0.2) (layer "B.Cu") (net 17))
 (segment (start 118.695 52.23) (end 116.68585 52.23) (width 0.2) (layer "B.Cu") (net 18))
 (segment (start 126.315 54.77) (end 121.235 54.77) (width 0.2) (layer "B.Cu") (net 18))
 (segment (start 128.181 40.54395) (end 128.181 44.399) (width 0.2) (layer "B.Cu") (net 18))
 (segment (start 116.68585 52.23) (end 113.998 49.54215) (width 0.2) (layer "B.Cu") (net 18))
 (segment (start 113.998 46.86495) (end 120.96395 39.899) (width 0.2) (layer "B.Cu") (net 18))
 (segment (start 120.96395 39.899) (end 127.53605 39.899) (width 0.2) (layer "B.Cu") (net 18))
 (segment (start 113.998 49.54215) (end 113.998 46.86495) (width 0.2) (layer "B.Cu") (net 18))
 (segment (start 118.75 62) (end 117.594 60.844) (width 0.2) (layer "B.Cu") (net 18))
 (segment (start 128.181 44.399) (end 127.08 45.5) (width 0.2) (layer "B.Cu") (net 18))
 (segment (start 121.235 54.77) (end 118.695 52.23) (width 0.2) (layer "B.Cu") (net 18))
 (segment (start 117.594 60.844) (end 117.594 53.331) (width 0.2) (layer "B.Cu") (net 18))
 (segment (start 117.594 53.331) (end 118.695 52.23) (width 0.2) (layer "B.Cu") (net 18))
 (segment (start 127.53605 39.899) (end 128.181 40.54395) (width 0.2) (layer "B.Cu") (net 18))
 (segment (start 129.459 45.43395) (end 129.459 42.89395) (width 0.2) (layer "F.Cu") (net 10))
 (segment (start 129.459 57.489) (end 129.459 45.43395) (width 0.2) (layer "F.Cu") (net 10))
 (segment (start 129.459 45.43395) (end 130.10395 44.789) (width 0.2) (layer "F.Cu") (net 10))
 (segment (start 129.459 42.89395) (end 130.35295 42) (width 0.2) (layer "F.Cu") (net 10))
 (segment (start 131.01605 44.789) (end 134.65705 48.43) (width 0.2) (layer "F.Cu") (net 10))
 (segment (start 130.56 58.59) (end 129.459 57.489) (width 0.2) (layer "F.Cu") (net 10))
 (segment (start 130.10395 44.789) (end 131.01605 44.789) (width 0.2) (layer "F.Cu") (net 10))
 (segment (start 134.65705 48.43) (end 138.18 48.43) (width 0.2) (layer "F.Cu") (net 10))
 (segment (start 130.35295 42) (end 131.1829 42) (width 0.2) (layer "F.Cu") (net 10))
 (segment (start 131.1829 42) (end 132.5329 43.35) (width 0.2) (layer "F.Cu") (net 10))
 (segment (start 132.5329 43.35) (end 138.18 43.35) (width 0.2) (layer "F.Cu") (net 10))
 (segment (start 127.58 63.33) (end 126.25 62) (width 0.2) (layer "B.Cu") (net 10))
 (segment (start 139.281 45.43395) (end 139.281 46.68405) (width 0.2) (layer "B.Cu") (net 10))
 (segment (start 132.64395 49.869) (end 137.72395 44.789) (width 0.2) (layer "B.Cu") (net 10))
 (segment (start 127.58 67.5) (end 127.58 63.33) (width 0.2) (layer "B.Cu") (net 10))
 (segment (start 120.134 51.129) (end 128.84395 51.129) (width 0.2) (layer "B.Cu") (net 10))
 (segment (start 130.10395 49.869) (end 132.64395 49.869) (width 0.2) (layer "B.Cu") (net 10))
 (segment (start 129 57.03) (end 130.56 58.59) (width 0.2) (layer "B.Cu") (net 10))
 (segment (start 129 56.05295) (end 129 57.03) (width 0.2) (layer "B.Cu") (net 10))
 (segment (start 136.933471 65.03) (end 136.933471 64.963471) (width 0.2) (layer "B.Cu") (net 10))
 (segment (start 137.72395 44.789) (end 138.63605 44.789) (width 0.2) (layer "B.Cu") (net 10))
 (segment (start 139.281 46.68405) (end 131.01605 54.949) (width 0.2) (layer "B.Cu") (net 10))
 (segment (start 115.5 48.92) (end 117.925 48.92) (width 0.2) (layer "B.Cu") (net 10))
 (segment (start 126.25 62) (end 122.25 66) (width 0.2) (layer "B.Cu") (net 10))
 (segment (start 131.01605 54.949) (end 130.10395 54.949) (width 0.2) (layer "B.Cu") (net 10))
 (segment (start 118.695 49.69) (end 120.134 51.129) (width 0.2) (layer "B.Cu") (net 10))
 (segment (start 130.451 66.201) (end 135.762471 66.201) (width 0.2) (layer "B.Cu") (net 10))
 (segment (start 135.762471 66.201) (end 136.933471 65.03) (width 0.2) (layer "B.Cu") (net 10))
 (segment (start 130.10395 54.949) (end 129 56.05295) (width 0.2) (layer "B.Cu") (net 10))
 (segment (start 122.25 66) (end 113 66) (width 0.2) (layer "B.Cu") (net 10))
 (segment (start 138.63605 44.789) (end 139.281 45.43395) (width 0.2) (layer "B.Cu") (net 10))
 (segment (start 136.933471 64.963471) (end 130.56 58.59) (width 0.2) (layer "B.Cu") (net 10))
 (segment (start 126.25 62) (end 130.451 66.201) (width 0.2) (layer "B.Cu") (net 10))
 (segment (start 128.84395 51.129) (end 130.10395 49.869) (width 0.2) (layer "B.Cu") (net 10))
 (segment (start 117.925 48.92) (end 118.695 49.69) (width 0.2) (layer "B.Cu") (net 10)))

